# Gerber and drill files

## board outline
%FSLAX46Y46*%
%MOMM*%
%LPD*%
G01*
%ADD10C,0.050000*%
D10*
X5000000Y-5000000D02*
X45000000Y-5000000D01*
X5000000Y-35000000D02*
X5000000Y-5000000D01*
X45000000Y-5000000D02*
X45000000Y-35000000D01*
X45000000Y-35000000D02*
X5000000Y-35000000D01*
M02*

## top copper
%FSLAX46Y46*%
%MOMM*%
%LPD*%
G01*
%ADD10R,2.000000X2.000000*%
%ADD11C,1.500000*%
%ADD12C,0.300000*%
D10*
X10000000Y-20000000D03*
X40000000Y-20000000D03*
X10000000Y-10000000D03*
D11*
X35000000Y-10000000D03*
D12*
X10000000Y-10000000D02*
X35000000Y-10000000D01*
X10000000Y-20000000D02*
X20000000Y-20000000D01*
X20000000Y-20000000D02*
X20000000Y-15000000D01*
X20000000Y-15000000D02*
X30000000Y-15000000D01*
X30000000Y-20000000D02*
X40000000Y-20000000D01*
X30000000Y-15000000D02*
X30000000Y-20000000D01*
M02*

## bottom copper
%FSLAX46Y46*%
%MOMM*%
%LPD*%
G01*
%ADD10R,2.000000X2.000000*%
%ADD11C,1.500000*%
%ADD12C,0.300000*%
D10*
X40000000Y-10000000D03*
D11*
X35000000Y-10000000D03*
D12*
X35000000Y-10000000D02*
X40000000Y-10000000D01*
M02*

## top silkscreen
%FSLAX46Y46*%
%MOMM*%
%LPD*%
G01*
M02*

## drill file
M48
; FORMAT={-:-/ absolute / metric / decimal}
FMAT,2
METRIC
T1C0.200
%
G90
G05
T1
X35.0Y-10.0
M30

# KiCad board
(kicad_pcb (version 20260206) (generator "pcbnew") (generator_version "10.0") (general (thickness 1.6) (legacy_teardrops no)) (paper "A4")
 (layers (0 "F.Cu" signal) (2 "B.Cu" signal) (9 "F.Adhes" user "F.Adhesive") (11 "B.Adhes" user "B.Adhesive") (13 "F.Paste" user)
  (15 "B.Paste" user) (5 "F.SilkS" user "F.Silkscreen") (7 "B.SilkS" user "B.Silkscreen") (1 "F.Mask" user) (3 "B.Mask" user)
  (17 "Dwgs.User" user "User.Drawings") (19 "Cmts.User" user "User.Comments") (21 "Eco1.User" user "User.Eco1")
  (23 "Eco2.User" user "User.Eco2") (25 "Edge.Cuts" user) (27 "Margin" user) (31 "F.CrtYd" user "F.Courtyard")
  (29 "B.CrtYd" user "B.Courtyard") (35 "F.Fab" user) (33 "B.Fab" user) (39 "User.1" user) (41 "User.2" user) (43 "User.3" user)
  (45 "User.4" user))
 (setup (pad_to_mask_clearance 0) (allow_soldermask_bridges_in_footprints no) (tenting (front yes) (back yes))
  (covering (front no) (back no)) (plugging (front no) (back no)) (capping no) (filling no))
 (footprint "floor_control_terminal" (layer "F.Cu") (at 10 20)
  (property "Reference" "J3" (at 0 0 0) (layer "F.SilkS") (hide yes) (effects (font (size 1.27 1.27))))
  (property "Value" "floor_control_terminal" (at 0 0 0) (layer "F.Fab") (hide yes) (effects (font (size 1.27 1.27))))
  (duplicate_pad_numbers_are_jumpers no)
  (pad "1" smd rect (at 0 0) (size 2 2) (layers "F.Cu" "F.Mask" "F.Paste") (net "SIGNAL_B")))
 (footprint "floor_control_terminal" (layer "F.Cu") (at 40 20)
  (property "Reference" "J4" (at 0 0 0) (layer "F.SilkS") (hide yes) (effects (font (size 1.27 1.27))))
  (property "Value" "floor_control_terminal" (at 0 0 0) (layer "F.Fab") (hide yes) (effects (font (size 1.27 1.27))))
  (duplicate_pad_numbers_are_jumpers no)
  (pad "1" smd rect (at 0 0) (size 2 2) (layers "F.Cu" "F.Mask" "F.Paste") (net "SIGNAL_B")))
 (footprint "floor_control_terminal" (layer "F.Cu") (at 10 10)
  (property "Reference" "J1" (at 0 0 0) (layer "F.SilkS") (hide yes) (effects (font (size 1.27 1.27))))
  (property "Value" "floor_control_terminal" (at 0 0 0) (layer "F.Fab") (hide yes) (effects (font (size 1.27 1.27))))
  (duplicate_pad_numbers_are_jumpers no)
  (pad "1" smd rect (at 0 0) (size 2 2) (layers "F.Cu" "F.Mask" "F.Paste") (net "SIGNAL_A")))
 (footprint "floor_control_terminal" (layer "B.Cu") (at 40 10)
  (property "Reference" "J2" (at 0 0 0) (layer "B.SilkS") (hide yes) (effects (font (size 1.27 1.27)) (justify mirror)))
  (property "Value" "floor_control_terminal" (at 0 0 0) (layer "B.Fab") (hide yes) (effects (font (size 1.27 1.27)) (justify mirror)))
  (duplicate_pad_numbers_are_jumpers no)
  (pad "1" smd rect (at 0 0) (size 2 2) (layers "B.Cu" "B.Mask" "B.Paste") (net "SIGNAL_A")))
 (gr_line (start 5 5) (end 45 5) (stroke (width 0.05) (type default)) (layer "Edge.Cuts"))
 (gr_line (start 5 35) (end 5 5) (stroke (width 0.05) (type default)) (layer "Edge.Cuts"))
 (gr_line (start 45 5) (end 45 35) (stroke (width 0.05) (type default)) (layer "Edge.Cuts"))
 (gr_line (start 45 35) (end 5 35) (stroke (width 0.05) (type default)) (layer "Edge.Cuts"))
 (segment (start 10 10) (end 35 10) (width 0.3) (layer "F.Cu") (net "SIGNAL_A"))
 (via (at 35 10) (size 1.5) (drill 0.2) (layers "F.Cu" "B.Cu") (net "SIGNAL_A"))
 (segment (start 35 10) (end 40 10) (width 0.3) (layer "B.Cu") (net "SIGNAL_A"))
 (segment (start 10 20) (end 20 20) (width 0.3) (layer "F.Cu") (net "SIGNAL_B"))
 (segment (start 20 20) (end 20 15) (width 0.3) (layer "F.Cu") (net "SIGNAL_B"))
 (segment (start 20 15) (end 30 15) (width 0.3) (layer "F.Cu") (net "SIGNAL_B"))
 (segment (start 30 20) (end 40 20) (width 0.3) (layer "F.Cu") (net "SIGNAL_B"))
 (segment (start 30 15) (end 30 20) (width 0.3) (layer "F.Cu") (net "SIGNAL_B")))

